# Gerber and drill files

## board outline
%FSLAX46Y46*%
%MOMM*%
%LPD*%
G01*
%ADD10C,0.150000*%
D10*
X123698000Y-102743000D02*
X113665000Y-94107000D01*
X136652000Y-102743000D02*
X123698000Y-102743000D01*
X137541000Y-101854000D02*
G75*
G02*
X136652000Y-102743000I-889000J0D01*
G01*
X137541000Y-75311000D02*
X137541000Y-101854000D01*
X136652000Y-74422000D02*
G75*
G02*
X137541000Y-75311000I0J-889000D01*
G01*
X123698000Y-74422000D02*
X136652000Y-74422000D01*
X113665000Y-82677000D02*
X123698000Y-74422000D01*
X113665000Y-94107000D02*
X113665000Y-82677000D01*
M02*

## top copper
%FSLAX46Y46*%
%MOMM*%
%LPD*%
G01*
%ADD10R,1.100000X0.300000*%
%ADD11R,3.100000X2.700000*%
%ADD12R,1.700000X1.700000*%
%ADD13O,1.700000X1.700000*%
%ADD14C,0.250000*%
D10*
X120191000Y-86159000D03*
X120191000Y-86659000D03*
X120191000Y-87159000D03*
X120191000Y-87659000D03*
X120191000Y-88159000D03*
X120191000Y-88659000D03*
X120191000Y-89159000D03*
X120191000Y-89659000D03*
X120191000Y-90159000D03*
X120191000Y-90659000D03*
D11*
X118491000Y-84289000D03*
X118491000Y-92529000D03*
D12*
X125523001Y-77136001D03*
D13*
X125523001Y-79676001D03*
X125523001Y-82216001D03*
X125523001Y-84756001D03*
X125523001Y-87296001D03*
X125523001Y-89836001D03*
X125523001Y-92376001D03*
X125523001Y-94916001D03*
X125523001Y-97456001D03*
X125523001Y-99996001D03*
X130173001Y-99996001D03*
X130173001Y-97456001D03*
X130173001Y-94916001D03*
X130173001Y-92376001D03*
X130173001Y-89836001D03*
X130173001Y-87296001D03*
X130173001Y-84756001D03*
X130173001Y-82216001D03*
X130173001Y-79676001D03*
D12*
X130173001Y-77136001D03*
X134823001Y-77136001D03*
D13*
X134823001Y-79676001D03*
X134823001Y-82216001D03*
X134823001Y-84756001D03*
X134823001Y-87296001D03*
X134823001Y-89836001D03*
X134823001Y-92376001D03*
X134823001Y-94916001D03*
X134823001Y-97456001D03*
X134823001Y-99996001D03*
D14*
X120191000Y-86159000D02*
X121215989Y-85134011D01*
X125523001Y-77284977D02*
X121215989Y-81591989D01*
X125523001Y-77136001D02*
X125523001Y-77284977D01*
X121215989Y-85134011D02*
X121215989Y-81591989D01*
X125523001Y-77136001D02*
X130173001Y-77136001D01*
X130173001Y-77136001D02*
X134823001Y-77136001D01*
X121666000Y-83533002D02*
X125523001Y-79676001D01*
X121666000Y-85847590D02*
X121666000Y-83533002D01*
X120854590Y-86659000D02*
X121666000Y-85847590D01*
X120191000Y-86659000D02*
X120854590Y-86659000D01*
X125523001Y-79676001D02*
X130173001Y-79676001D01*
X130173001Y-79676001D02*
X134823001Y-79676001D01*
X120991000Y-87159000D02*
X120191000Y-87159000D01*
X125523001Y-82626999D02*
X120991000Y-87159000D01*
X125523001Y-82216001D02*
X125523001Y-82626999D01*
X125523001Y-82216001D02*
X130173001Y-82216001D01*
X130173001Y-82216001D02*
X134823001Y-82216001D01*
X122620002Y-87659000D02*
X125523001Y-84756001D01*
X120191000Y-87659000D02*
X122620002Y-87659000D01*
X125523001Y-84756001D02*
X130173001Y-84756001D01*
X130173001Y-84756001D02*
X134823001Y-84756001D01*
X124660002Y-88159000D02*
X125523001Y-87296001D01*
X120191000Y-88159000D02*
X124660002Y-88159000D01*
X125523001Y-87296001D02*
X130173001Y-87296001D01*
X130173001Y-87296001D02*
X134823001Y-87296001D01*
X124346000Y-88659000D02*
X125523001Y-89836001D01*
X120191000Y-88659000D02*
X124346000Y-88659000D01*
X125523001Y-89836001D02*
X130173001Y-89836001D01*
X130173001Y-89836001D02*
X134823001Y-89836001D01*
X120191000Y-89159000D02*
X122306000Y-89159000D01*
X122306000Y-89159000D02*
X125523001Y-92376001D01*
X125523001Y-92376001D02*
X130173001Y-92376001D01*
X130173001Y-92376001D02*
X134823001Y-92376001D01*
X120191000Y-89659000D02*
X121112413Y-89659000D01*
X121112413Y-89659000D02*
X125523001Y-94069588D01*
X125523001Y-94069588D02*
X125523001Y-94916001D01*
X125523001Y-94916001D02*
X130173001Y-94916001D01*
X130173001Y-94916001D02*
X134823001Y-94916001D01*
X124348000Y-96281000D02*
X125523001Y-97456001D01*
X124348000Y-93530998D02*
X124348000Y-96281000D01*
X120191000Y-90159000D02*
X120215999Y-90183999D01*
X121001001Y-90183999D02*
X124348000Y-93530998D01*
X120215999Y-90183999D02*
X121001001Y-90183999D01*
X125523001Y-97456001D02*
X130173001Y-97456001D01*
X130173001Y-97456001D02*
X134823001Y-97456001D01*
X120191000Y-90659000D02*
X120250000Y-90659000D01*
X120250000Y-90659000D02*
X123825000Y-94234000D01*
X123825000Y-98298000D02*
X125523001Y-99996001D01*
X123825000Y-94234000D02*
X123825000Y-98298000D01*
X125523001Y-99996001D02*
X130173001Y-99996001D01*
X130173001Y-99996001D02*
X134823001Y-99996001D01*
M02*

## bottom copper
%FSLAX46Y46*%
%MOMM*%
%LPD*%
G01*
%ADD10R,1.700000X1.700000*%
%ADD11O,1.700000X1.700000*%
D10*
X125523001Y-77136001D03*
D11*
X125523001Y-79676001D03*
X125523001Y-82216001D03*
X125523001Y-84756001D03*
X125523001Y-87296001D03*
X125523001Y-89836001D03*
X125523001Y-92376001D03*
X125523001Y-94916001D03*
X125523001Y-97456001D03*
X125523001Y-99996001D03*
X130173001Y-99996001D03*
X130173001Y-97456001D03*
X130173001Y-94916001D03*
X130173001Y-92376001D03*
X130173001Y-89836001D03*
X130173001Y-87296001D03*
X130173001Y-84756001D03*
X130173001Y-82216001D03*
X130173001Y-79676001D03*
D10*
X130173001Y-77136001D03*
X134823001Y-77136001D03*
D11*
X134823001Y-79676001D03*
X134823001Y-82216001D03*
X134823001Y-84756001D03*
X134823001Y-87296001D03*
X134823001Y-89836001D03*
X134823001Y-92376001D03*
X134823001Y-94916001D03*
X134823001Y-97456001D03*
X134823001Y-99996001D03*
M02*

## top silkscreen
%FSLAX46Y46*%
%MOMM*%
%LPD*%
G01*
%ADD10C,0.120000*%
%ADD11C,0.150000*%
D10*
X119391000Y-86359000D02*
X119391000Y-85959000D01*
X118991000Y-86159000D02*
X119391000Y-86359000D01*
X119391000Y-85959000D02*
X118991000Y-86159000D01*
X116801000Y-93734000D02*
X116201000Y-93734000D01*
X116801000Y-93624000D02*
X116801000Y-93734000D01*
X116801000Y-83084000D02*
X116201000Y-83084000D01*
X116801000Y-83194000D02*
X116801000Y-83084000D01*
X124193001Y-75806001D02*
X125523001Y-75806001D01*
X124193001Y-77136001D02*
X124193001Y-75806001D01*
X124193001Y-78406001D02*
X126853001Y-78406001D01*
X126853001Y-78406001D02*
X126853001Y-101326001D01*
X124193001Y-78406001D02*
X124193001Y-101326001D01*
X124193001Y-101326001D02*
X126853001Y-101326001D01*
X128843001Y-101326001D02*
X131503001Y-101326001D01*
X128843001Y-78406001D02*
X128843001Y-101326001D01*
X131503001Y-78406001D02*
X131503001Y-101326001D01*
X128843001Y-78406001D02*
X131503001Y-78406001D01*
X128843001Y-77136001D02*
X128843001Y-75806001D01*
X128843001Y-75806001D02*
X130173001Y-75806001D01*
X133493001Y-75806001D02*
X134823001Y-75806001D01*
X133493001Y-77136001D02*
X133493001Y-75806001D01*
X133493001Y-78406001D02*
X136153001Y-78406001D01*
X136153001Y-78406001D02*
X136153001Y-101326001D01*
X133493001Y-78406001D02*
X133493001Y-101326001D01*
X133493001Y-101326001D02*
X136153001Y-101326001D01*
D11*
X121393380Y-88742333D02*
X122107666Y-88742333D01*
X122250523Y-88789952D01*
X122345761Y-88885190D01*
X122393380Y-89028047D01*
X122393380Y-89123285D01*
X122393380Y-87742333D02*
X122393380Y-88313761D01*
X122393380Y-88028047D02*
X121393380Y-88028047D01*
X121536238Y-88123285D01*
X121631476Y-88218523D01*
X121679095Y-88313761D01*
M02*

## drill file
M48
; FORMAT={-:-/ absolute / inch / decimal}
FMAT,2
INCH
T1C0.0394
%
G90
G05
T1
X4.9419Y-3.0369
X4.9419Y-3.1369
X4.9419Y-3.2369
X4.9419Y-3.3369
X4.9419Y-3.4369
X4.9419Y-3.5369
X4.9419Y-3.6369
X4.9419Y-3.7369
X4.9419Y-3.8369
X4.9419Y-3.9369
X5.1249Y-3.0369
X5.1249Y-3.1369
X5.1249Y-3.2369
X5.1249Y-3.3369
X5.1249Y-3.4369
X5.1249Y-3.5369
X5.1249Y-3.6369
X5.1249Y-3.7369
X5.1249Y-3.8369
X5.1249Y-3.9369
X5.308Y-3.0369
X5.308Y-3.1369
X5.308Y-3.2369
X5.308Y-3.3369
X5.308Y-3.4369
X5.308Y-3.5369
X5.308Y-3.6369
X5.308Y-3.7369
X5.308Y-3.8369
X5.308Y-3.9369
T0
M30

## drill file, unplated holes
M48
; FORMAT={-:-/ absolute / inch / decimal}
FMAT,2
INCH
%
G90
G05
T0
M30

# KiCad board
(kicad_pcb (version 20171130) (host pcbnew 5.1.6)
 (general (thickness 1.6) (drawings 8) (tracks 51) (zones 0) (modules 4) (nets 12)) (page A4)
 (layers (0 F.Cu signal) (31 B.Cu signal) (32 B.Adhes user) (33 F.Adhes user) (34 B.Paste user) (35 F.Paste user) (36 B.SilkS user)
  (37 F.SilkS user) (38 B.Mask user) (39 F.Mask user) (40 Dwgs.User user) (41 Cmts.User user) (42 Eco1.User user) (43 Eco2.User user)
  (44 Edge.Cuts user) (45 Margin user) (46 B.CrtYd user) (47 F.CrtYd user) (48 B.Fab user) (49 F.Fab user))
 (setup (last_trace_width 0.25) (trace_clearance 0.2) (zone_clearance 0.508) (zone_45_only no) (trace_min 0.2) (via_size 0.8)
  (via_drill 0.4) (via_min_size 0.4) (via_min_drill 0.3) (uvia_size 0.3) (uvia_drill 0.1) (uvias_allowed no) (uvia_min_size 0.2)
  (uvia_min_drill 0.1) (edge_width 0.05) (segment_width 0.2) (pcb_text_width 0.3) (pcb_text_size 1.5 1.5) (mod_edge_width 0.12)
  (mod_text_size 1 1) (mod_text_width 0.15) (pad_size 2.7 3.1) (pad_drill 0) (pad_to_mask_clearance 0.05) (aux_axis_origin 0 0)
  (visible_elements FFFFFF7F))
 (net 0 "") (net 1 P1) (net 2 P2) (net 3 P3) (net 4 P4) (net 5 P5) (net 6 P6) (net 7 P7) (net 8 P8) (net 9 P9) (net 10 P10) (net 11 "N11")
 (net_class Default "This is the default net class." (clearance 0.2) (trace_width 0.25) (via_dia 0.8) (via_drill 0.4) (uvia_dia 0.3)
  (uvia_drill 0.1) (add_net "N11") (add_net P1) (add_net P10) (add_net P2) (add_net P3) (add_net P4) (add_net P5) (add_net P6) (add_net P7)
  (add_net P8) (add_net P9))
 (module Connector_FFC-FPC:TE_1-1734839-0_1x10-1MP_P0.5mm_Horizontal (layer F.Cu) (at 118.841 88.409 270)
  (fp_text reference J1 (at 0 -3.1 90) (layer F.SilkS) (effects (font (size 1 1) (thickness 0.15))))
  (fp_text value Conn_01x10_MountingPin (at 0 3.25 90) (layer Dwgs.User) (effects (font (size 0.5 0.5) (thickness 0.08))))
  (fp_line (start -2.05 -0.55) (end -2.45 -0.55) (layer F.SilkS) (width 0.12))
  (fp_line (start -2.25 -0.15) (end -2.05 -0.55) (layer F.SilkS) (width 0.12))
  (fp_line (start -2.45 -0.55) (end -2.25 -0.15) (layer F.SilkS) (width 0.12))
  (fp_line (start 5.325 2.04) (end 5.325 2.64) (layer F.SilkS) (width 0.12))
  (fp_line (start 5.215 2.04) (end 5.325 2.04) (layer F.SilkS) (width 0.12))
  (fp_line (start -5.325 2.04) (end -5.325 2.64) (layer F.SilkS) (width 0.12))
  (fp_line (start -5.215 2.04) (end -5.325 2.04) (layer F.SilkS) (width 0.12))
  (pad 1 smd rect (at -2.25 -1.35 270) (size 0.3 1.1) (layers F.Cu F.Paste F.Mask) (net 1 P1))
  (pad 2 smd rect (at -1.75 -1.35 270) (size 0.3 1.1) (layers F.Cu F.Paste F.Mask) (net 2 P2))
  (pad 3 smd rect (at -1.25 -1.35 270) (size 0.3 1.1) (layers F.Cu F.Paste F.Mask) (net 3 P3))
  (pad 4 smd rect (at -0.75 -1.35 270) (size 0.3 1.1) (layers F.Cu F.Paste F.Mask) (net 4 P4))
  (pad 5 smd rect (at -0.25 -1.35 270) (size 0.3 1.1) (layers F.Cu F.Paste F.Mask) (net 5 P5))
  (pad 6 smd rect (at 0.25 -1.35 270) (size 0.3 1.1) (layers F.Cu F.Paste F.Mask) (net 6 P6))
  (pad 7 smd rect (at 0.75 -1.35 270) (size 0.3 1.1) (layers F.Cu F.Paste F.Mask) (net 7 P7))
  (pad 8 smd rect (at 1.25 -1.35 270) (size 0.3 1.1) (layers F.Cu F.Paste F.Mask) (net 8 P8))
  (pad 9 smd rect (at 1.75 -1.35 270) (size 0.3 1.1) (layers F.Cu F.Paste F.Mask) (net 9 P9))
  (pad 10 smd rect (at 2.25 -1.35 270) (size 0.3 1.1) (layers F.Cu F.Paste F.Mask) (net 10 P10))
  (pad MP smd rect (at -4.12 0.35 270) (size 2.7 3.1) (layers F.Cu F.Paste F.Mask) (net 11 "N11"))
  (pad MP smd rect (at 4.12 0.35 270) (size 2.7 3.1) (layers F.Cu F.Paste F.Mask) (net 11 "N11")))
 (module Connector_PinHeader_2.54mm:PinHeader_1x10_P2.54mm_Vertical (layer F.Cu) (at 125.523001 77.136001)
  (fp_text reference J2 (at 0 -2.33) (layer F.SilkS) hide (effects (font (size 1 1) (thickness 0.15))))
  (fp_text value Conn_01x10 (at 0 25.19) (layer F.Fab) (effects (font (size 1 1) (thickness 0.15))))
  (fp_line (start -1.33 -1.33) (end 0 -1.33) (layer F.SilkS) (width 0.12))
  (fp_line (start -1.33 0) (end -1.33 -1.33) (layer F.SilkS) (width 0.12))
  (fp_line (start -1.33 1.27) (end 1.33 1.27) (layer F.SilkS) (width 0.12))
  (fp_line (start 1.33 1.27) (end 1.33 24.19) (layer F.SilkS) (width 0.12))
  (fp_line (start -1.33 1.27) (end -1.33 24.19) (layer F.SilkS) (width 0.12))
  (fp_line (start -1.33 24.19) (end 1.33 24.19) (layer F.SilkS) (width 0.12))
  (pad 1 thru_hole rect (at 0 0) (size 1.7 1.7) (drill 1) (layers *.Cu *.Mask) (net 1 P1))
  (pad 2 thru_hole oval (at 0 2.54) (size 1.7 1.7) (drill 1) (layers *.Cu *.Mask) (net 2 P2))
  (pad 3 thru_hole oval (at 0 5.08) (size 1.7 1.7) (drill 1) (layers *.Cu *.Mask) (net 3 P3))
  (pad 4 thru_hole oval (at 0 7.62) (size 1.7 1.7) (drill 1) (layers *.Cu *.Mask) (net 4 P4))
  (pad 5 thru_hole oval (at 0 10.16) (size 1.7 1.7) (drill 1) (layers *.Cu *.Mask) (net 5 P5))
  (pad 6 thru_hole oval (at 0 12.7) (size 1.7 1.7) (drill 1) (layers *.Cu *.Mask) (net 6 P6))
  (pad 7 thru_hole oval (at 0 15.24) (size 1.7 1.7) (drill 1) (layers *.Cu *.Mask) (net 7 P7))
  (pad 8 thru_hole oval (at 0 17.78) (size 1.7 1.7) (drill 1) (layers *.Cu *.Mask) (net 8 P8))
  (pad 9 thru_hole oval (at 0 20.32) (size 1.7 1.7) (drill 1) (layers *.Cu *.Mask) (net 9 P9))
  (pad 10 thru_hole oval (at 0 22.86) (size 1.7 1.7) (drill 1) (layers *.Cu *.Mask) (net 10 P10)))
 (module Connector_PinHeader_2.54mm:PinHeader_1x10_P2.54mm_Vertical (layer F.Cu) (at 130.173001 77.136001)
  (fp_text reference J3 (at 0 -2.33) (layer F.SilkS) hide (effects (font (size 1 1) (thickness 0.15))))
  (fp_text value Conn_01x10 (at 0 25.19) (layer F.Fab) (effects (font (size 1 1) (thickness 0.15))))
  (fp_line (start -1.33 24.19) (end 1.33 24.19) (layer F.SilkS) (width 0.12))
  (fp_line (start -1.33 1.27) (end -1.33 24.19) (layer F.SilkS) (width 0.12))
  (fp_line (start 1.33 1.27) (end 1.33 24.19) (layer F.SilkS) (width 0.12))
  (fp_line (start -1.33 1.27) (end 1.33 1.27) (layer F.SilkS) (width 0.12))
  (fp_line (start -1.33 0) (end -1.33 -1.33) (layer F.SilkS) (width 0.12))
  (fp_line (start -1.33 -1.33) (end 0 -1.33) (layer F.SilkS) (width 0.12))
  (pad 10 thru_hole oval (at 0 22.86) (size 1.7 1.7) (drill 1) (layers *.Cu *.Mask) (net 10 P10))
  (pad 9 thru_hole oval (at 0 20.32) (size 1.7 1.7) (drill 1) (layers *.Cu *.Mask) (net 9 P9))
  (pad 8 thru_hole oval (at 0 17.78) (size 1.7 1.7) (drill 1) (layers *.Cu *.Mask) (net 8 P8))
  (pad 7 thru_hole oval (at 0 15.24) (size 1.7 1.7) (drill 1) (layers *.Cu *.Mask) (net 7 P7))
  (pad 6 thru_hole oval (at 0 12.7) (size 1.7 1.7) (drill 1) (layers *.Cu *.Mask) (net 6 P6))
  (pad 5 thru_hole oval (at 0 10.16) (size 1.7 1.7) (drill 1) (layers *.Cu *.Mask) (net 5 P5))
  (pad 4 thru_hole oval (at 0 7.62) (size 1.7 1.7) (drill 1) (layers *.Cu *.Mask) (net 4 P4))
  (pad 3 thru_hole oval (at 0 5.08) (size 1.7 1.7) (drill 1) (layers *.Cu *.Mask) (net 3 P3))
  (pad 2 thru_hole oval (at 0 2.54) (size 1.7 1.7) (drill 1) (layers *.Cu *.Mask) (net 2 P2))
  (pad 1 thru_hole rect (at 0 0) (size 1.7 1.7) (drill 1) (layers *.Cu *.Mask) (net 1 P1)))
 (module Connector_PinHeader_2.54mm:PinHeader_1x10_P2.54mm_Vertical (layer F.Cu) (at 134.823001 77.136001)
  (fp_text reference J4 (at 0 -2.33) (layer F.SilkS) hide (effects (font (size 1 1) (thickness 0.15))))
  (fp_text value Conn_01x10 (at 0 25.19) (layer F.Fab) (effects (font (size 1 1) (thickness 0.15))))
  (fp_line (start -1.33 -1.33) (end 0 -1.33) (layer F.SilkS) (width 0.12))
  (fp_line (start -1.33 0) (end -1.33 -1.33) (layer F.SilkS) (width 0.12))
  (fp_line (start -1.33 1.27) (end 1.33 1.27) (layer F.SilkS) (width 0.12))
  (fp_line (start 1.33 1.27) (end 1.33 24.19) (layer F.SilkS) (width 0.12))
  (fp_line (start -1.33 1.27) (end -1.33 24.19) (layer F.SilkS) (width 0.12))
  (fp_line (start -1.33 24.19) (end 1.33 24.19) (layer F.SilkS) (width 0.12))
  (pad 1 thru_hole rect (at 0 0) (size 1.7 1.7) (drill 1) (layers *.Cu *.Mask) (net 1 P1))
  (pad 2 thru_hole oval (at 0 2.54) (size 1.7 1.7) (drill 1) (layers *.Cu *.Mask) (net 2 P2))
  (pad 3 thru_hole oval (at 0 5.08) (size 1.7 1.7) (drill 1) (layers *.Cu *.Mask) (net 3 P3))
  (pad 4 thru_hole oval (at 0 7.62) (size 1.7 1.7) (drill 1) (layers *.Cu *.Mask) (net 4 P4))
  (pad 5 thru_hole oval (at 0 10.16) (size 1.7 1.7) (drill 1) (layers *.Cu *.Mask) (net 5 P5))
  (pad 6 thru_hole oval (at 0 12.7) (size 1.7 1.7) (drill 1) (layers *.Cu *.Mask) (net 6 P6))
  (pad 7 thru_hole oval (at 0 15.24) (size 1.7 1.7) (drill 1) (layers *.Cu *.Mask) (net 7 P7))
  (pad 8 thru_hole oval (at 0 17.78) (size 1.7 1.7) (drill 1) (layers *.Cu *.Mask) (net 8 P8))
  (pad 9 thru_hole oval (at 0 20.32) (size 1.7 1.7) (drill 1) (layers *.Cu *.Mask) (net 9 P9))
  (pad 10 thru_hole oval (at 0 22.86) (size 1.7 1.7) (drill 1) (layers *.Cu *.Mask) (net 10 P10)))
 (gr_line (start 123.698 102.743) (end 113.665 94.107) (layer Edge.Cuts) (width 0.15))
 (gr_line (start 136.652 102.743) (end 123.698 102.743) (layer Edge.Cuts) (width 0.15))
 (gr_arc (start 136.652 101.854) (end 136.652 102.743) (angle -90) (layer Edge.Cuts) (width 0.15))
 (gr_line (start 137.541 75.311) (end 137.541 101.854) (layer Edge.Cuts) (width 0.15))
 (gr_arc (start 136.652 75.311) (end 137.541 75.311) (angle -90) (layer Edge.Cuts) (width 0.15))
 (gr_line (start 123.698 74.422) (end 136.652 74.422) (layer Edge.Cuts) (width 0.15))
 (gr_line (start 113.665 82.677) (end 123.698 74.422) (layer Edge.Cuts) (width 0.15))
 (gr_line (start 113.665 94.107) (end 113.665 82.677) (layer Edge.Cuts) (width 0.15))
 (segment (start 120.191 86.159) (end 121.215989 85.134011) (width 0.25) (layer F.Cu) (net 1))
 (segment (start 125.523001 77.284977) (end 121.215989 81.591989) (width 0.25) (layer F.Cu) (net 1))
 (segment (start 125.523001 77.136001) (end 125.523001 77.284977) (width 0.25) (layer F.Cu) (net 1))
 (segment (start 121.215989 85.134011) (end 121.215989 81.591989) (width 0.25) (layer F.Cu) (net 1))
 (segment (start 125.523001 77.136001) (end 130.173001 77.136001) (width 0.25) (layer F.Cu) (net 1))
 (segment (start 130.173001 77.136001) (end 134.823001 77.136001) (width 0.25) (layer F.Cu) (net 1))
 (segment (start 121.666 83.533002) (end 125.523001 79.676001) (width 0.25) (layer F.Cu) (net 2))
 (segment (start 121.666 85.84759) (end 121.666 83.533002) (width 0.25) (layer F.Cu) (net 2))
 (segment (start 120.85459 86.659) (end 121.666 85.84759) (width 0.25) (layer F.Cu) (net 2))
 (segment (start 120.191 86.659) (end 120.85459 86.659) (width 0.25) (layer F.Cu) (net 2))
 (segment (start 125.523001 79.676001) (end 130.173001 79.676001) (width 0.25) (layer F.Cu) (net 2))
 (segment (start 130.173001 79.676001) (end 134.823001 79.676001) (width 0.25) (layer F.Cu) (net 2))
 (segment (start 120.991 87.159) (end 120.191 87.159) (width 0.25) (layer F.Cu) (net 3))
 (segment (start 125.523001 82.626999) (end 120.991 87.159) (width 0.25) (layer F.Cu) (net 3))
 (segment (start 125.523001 82.216001) (end 125.523001 82.626999) (width 0.25) (layer F.Cu) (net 3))
 (segment (start 125.523001 82.216001) (end 130.173001 82.216001) (width 0.25) (layer F.Cu) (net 3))
 (segment (start 130.173001 82.216001) (end 134.823001 82.216001) (width 0.25) (layer F.Cu) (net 3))
 (segment (start 122.620002 87.659) (end 125.523001 84.756001) (width 0.25) (layer F.Cu) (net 4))
 (segment (start 120.191 87.659) (end 122.620002 87.659) (width 0.25) (layer F.Cu) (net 4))
 (segment (start 125.523001 84.756001) (end 130.173001 84.756001) (width 0.25) (layer F.Cu) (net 4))
 (segment (start 130.173001 84.756001) (end 134.823001 84.756001) (width 0.25) (layer F.Cu) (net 4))
 (segment (start 124.660002 88.159) (end 125.523001 87.296001) (width 0.25) (layer F.Cu) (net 5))
 (segment (start 120.191 88.159) (end 124.660002 88.159) (width 0.25) (layer F.Cu) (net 5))
 (segment (start 125.523001 87.296001) (end 130.173001 87.296001) (width 0.25) (layer F.Cu) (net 5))
 (segment (start 130.173001 87.296001) (end 134.823001 87.296001) (width 0.25) (layer F.Cu) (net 5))
 (segment (start 124.346 88.659) (end 125.523001 89.836001) (width 0.25) (layer F.Cu) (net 6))
 (segment (start 120.191 88.659) (end 124.346 88.659) (width 0.25) (layer F.Cu) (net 6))
 (segment (start 125.523001 89.836001) (end 130.173001 89.836001) (width 0.25) (layer F.Cu) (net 6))
 (segment (start 130.173001 89.836001) (end 134.823001 89.836001) (width 0.25) (layer F.Cu) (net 6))
 (segment (start 120.191 89.159) (end 122.306 89.159) (width 0.25) (layer F.Cu) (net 7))
 (segment (start 122.306 89.159) (end 125.523001 92.376001) (width 0.25) (layer F.Cu) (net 7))
 (segment (start 125.523001 92.376001) (end 130.173001 92.376001) (width 0.25) (layer F.Cu) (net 7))
 (segment (start 130.173001 92.376001) (end 134.823001 92.376001) (width 0.25) (layer F.Cu) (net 7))
 (segment (start 120.191 89.659) (end 121.112413 89.659) (width 0.25) (layer F.Cu) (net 8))
 (segment (start 121.112413 89.659) (end 125.523001 94.069588) (width 0.25) (layer F.Cu) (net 8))
 (segment (start 125.523001 94.069588) (end 125.523001 94.916001) (width 0.25) (layer F.Cu) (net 8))
 (segment (start 125.523001 94.916001) (end 130.173001 94.916001) (width 0.25) (layer F.Cu) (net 8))
 (segment (start 130.173001 94.916001) (end 134.823001 94.916001) (width 0.25) (layer F.Cu) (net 8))
 (segment (start 124.348 96.281) (end 125.523001 97.456001) (width 0.25) (layer F.Cu) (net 9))
 (segment (start 124.348 93.530998) (end 124.348 96.281) (width 0.25) (layer F.Cu) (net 9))
 (segment (start 120.191 90.159) (end 120.215999 90.183999) (width 0.25) (layer F.Cu) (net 9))
 (segment (start 121.001001 90.183999) (end 124.348 93.530998) (width 0.25) (layer F.Cu) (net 9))
 (segment (start 120.215999 90.183999) (end 121.001001 90.183999) (width 0.25) (layer F.Cu) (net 9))
 (segment (start 125.523001 97.456001) (end 130.173001 97.456001) (width 0.25) (layer F.Cu) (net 9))
 (segment (start 130.173001 97.456001) (end 134.823001 97.456001) (width 0.25) (layer F.Cu) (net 9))
 (segment (start 120.191 90.659) (end 120.25 90.659) (width 0.25) (layer F.Cu) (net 10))
 (segment (start 120.25 90.659) (end 123.825 94.234) (width 0.25) (layer F.Cu) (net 10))
 (segment (start 123.825 98.298) (end 125.523001 99.996001) (width 0.25) (layer F.Cu) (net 10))
 (segment (start 123.825 94.234) (end 123.825 98.298) (width 0.25) (layer F.Cu) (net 10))
 (segment (start 125.523001 99.996001) (end 130.173001 99.996001) (width 0.25) (layer F.Cu) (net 10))
 (segment (start 130.173001 99.996001) (end 134.823001 99.996001) (width 0.25) (layer F.Cu) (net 10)))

